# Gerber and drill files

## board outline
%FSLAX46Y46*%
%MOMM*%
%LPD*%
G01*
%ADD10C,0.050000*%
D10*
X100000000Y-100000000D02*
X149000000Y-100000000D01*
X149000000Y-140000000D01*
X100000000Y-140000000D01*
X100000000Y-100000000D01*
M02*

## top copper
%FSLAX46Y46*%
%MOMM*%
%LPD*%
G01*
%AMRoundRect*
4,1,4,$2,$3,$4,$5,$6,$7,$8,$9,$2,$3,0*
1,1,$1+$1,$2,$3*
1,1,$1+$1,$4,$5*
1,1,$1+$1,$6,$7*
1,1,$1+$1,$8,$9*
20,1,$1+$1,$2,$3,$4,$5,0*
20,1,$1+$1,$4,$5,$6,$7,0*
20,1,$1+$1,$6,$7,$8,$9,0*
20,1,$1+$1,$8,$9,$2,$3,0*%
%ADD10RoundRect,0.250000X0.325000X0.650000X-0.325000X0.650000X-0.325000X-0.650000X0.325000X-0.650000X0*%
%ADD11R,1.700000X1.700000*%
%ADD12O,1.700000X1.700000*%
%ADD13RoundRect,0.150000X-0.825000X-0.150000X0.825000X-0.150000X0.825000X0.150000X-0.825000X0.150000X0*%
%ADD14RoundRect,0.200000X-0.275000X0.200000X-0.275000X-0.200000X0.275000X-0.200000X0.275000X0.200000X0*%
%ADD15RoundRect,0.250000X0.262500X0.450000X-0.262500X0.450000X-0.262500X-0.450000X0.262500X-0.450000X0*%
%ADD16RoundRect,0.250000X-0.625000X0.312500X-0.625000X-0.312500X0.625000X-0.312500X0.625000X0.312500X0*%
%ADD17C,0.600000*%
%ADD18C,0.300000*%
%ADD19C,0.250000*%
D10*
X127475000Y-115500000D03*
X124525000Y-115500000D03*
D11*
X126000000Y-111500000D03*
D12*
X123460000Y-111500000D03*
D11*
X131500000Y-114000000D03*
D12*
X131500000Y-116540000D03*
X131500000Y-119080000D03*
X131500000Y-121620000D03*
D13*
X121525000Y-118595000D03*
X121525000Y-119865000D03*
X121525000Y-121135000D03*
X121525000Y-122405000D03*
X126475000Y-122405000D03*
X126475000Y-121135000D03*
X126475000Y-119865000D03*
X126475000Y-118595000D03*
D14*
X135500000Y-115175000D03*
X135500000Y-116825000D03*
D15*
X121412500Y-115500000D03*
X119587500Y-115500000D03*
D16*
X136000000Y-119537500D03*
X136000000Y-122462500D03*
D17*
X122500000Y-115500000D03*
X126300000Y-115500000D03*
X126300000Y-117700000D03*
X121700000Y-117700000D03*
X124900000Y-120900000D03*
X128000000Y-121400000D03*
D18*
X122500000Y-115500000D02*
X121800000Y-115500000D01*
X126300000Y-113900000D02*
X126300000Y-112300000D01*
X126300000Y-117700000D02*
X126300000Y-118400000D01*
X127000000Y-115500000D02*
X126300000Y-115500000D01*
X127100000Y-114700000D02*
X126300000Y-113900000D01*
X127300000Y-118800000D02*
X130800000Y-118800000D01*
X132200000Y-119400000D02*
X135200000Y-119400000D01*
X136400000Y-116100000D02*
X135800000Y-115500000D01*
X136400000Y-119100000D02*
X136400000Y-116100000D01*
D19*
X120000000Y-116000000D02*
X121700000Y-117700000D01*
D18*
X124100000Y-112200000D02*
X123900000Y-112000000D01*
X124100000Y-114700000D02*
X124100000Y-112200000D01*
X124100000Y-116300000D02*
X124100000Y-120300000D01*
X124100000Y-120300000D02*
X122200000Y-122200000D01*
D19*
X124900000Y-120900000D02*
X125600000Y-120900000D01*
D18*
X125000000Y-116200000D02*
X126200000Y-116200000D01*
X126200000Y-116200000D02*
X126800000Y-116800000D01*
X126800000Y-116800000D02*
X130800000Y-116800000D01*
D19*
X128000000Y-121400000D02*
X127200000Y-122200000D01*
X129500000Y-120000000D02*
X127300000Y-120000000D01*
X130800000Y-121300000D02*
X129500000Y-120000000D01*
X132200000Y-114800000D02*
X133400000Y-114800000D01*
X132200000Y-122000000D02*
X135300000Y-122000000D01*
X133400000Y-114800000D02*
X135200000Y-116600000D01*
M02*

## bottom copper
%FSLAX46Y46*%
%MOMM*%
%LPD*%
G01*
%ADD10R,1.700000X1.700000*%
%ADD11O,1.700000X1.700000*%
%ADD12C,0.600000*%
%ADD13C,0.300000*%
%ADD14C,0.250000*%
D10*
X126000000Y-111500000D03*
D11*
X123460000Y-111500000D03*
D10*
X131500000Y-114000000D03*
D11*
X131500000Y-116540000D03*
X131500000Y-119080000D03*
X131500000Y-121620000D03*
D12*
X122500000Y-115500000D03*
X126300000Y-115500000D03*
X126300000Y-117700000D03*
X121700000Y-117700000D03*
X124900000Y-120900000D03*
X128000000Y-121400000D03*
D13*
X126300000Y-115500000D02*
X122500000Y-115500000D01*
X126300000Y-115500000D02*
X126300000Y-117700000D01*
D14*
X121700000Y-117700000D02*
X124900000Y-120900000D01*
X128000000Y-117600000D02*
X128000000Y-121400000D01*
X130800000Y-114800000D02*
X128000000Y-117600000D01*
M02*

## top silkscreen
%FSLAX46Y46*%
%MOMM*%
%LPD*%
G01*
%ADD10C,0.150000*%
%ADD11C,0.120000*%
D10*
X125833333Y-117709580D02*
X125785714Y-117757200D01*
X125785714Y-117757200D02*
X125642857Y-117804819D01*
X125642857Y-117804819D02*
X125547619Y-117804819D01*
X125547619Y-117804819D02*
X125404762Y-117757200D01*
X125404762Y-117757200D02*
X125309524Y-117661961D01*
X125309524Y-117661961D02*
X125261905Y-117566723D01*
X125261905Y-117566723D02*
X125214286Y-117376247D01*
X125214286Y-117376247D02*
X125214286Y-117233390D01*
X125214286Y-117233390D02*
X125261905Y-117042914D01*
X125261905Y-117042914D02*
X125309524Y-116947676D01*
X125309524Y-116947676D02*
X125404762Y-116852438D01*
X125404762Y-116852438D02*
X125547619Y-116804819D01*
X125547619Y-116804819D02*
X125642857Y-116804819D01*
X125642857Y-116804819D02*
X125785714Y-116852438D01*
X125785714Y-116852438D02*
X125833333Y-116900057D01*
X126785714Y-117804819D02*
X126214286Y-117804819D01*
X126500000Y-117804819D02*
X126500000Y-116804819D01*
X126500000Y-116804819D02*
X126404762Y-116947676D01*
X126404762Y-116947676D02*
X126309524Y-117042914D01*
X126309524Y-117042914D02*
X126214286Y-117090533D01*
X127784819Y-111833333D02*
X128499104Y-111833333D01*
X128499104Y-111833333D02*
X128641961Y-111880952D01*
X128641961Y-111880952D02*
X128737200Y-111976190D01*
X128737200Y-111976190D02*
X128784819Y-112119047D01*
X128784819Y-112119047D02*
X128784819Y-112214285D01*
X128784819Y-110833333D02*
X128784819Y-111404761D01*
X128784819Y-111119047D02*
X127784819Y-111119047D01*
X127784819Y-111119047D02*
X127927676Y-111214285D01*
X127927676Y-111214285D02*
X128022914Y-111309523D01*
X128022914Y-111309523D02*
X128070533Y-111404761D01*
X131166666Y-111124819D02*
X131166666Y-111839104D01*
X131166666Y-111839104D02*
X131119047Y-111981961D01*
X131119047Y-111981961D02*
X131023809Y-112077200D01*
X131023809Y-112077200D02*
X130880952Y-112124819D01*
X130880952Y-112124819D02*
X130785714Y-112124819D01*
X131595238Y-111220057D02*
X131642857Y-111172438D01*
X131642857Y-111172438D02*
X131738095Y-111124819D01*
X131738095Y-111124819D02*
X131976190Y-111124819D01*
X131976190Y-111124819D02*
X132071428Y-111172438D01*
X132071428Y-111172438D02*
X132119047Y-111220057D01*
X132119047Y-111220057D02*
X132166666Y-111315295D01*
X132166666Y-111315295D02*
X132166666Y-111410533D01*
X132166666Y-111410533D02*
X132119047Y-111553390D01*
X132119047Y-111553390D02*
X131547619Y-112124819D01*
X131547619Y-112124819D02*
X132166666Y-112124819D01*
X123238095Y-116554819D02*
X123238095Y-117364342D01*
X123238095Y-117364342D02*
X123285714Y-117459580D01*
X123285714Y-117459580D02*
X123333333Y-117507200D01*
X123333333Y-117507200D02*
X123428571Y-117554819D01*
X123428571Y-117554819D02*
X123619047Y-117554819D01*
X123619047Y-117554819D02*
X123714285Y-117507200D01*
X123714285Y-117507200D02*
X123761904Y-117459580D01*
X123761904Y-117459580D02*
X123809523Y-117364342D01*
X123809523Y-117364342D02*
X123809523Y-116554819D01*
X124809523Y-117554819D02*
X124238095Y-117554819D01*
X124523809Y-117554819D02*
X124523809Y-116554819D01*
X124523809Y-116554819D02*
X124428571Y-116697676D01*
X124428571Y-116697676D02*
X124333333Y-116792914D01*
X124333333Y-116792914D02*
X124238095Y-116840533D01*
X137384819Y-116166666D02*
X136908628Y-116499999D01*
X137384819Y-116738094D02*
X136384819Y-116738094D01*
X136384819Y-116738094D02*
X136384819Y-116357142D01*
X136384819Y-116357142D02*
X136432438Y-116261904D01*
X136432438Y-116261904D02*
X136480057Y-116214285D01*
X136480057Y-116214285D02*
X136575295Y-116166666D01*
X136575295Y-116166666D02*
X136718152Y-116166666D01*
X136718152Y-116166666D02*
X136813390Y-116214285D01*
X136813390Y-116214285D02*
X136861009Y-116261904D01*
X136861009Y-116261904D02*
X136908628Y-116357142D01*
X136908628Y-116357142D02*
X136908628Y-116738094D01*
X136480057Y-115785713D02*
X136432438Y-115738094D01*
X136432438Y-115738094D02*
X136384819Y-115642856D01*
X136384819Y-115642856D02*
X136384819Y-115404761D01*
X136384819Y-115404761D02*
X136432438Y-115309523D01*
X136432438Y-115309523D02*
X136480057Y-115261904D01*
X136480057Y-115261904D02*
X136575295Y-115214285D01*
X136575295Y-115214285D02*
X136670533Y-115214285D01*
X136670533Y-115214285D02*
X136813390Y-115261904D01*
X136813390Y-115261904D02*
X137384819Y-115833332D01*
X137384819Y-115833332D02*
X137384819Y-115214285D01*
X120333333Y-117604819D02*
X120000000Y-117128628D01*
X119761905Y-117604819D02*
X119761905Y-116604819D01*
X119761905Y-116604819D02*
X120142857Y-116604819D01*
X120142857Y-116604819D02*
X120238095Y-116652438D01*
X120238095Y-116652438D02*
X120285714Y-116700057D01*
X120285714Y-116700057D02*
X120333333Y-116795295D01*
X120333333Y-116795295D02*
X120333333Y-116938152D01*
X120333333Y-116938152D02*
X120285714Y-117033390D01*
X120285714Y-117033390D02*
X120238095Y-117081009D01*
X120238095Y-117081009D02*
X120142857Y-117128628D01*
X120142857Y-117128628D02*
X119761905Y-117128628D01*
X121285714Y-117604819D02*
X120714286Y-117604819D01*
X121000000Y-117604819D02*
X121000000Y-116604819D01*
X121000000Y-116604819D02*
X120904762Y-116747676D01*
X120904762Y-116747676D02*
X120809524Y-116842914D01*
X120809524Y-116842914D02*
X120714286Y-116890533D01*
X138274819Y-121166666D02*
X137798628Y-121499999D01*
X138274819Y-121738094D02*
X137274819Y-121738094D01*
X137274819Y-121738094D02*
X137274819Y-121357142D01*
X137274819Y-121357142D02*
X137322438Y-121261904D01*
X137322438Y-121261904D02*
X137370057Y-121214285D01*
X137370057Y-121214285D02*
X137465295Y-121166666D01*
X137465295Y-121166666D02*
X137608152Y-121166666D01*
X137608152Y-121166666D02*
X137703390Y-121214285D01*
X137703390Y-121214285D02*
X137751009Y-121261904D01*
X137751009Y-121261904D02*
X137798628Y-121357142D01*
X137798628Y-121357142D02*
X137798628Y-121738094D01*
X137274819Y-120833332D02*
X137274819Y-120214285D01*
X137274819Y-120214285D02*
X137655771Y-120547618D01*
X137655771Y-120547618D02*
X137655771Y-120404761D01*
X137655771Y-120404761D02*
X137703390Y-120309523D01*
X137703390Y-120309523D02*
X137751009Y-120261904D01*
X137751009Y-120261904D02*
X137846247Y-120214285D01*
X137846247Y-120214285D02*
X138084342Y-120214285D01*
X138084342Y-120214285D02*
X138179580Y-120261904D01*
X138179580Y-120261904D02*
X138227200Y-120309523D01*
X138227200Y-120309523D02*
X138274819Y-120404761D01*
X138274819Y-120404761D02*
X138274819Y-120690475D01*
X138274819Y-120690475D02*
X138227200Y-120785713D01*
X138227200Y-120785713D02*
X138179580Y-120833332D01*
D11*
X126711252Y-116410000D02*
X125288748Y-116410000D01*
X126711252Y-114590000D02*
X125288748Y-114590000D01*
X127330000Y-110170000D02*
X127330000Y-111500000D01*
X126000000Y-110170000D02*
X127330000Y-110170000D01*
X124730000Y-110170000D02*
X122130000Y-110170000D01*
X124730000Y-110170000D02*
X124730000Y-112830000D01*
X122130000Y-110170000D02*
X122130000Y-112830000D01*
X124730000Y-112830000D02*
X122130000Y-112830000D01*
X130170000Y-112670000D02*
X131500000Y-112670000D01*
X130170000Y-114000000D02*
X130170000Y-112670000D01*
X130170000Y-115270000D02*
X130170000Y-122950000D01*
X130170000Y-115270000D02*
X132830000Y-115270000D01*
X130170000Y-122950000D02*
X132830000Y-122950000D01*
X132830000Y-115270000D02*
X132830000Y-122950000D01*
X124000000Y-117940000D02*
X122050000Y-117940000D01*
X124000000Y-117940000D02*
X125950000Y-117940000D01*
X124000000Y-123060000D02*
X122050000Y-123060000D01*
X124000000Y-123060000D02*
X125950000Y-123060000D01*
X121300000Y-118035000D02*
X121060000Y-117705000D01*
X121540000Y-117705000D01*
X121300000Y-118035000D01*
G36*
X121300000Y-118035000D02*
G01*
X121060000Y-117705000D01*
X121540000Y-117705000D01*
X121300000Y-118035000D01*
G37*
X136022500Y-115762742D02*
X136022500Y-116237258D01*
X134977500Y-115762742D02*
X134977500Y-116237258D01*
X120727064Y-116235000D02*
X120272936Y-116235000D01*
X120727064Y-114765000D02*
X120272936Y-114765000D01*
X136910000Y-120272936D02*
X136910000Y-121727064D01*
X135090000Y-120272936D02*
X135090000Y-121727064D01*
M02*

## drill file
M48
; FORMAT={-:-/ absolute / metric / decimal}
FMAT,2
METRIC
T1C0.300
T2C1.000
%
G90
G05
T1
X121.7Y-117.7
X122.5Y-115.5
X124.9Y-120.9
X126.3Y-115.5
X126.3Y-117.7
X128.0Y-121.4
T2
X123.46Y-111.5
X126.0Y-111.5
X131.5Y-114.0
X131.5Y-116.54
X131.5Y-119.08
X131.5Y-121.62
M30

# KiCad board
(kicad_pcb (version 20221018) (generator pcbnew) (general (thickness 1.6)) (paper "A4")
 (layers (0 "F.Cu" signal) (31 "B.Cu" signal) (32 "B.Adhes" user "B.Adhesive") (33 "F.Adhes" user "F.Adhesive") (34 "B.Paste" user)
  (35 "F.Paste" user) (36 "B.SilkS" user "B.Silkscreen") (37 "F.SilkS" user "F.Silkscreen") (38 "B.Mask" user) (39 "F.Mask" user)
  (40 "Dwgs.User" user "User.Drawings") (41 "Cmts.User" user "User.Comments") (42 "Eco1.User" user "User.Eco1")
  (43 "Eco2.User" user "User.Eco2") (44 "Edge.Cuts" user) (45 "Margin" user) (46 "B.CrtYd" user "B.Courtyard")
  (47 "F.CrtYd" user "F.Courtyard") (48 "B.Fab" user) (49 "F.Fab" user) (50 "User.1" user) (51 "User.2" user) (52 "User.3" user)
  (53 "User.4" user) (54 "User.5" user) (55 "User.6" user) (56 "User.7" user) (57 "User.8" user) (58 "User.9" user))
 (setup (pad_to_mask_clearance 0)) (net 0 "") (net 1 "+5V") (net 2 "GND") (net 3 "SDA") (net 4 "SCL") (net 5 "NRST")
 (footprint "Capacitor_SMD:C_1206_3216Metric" (layer "F.Cu") (at 126 115.5 180)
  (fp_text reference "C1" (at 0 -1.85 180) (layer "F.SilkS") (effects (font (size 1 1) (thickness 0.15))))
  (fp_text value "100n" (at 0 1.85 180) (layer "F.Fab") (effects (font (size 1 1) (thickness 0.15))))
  (fp_line (start -0.711252 -0.91) (end 0.711252 -0.91) (stroke (width 0.12) (type solid)) (layer "F.SilkS"))
  (fp_line (start -0.711252 0.91) (end 0.711252 0.91) (stroke (width 0.12) (type solid)) (layer "F.SilkS"))
  (pad "1" smd roundrect (at -1.475 0 180) (size 1.15 1.8) (layers "F.Cu" "F.Paste" "F.Mask") (roundrect_rratio 0.217391) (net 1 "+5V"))
  (pad "2" smd roundrect (at 1.475 0 180) (size 1.15 1.8) (layers "F.Cu" "F.Paste" "F.Mask") (roundrect_rratio 0.217391) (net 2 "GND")))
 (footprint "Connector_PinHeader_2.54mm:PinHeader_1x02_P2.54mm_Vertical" (layer "F.Cu") (at 126 111.5 -90)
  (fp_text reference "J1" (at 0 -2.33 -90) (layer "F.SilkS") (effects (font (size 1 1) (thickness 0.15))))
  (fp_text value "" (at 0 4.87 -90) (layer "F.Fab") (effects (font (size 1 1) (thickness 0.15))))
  (fp_line (start -1.33 -1.33) (end 0 -1.33) (stroke (width 0.12) (type solid)) (layer "F.SilkS"))
  (fp_line (start -1.33 0) (end -1.33 -1.33) (stroke (width 0.12) (type solid)) (layer "F.SilkS"))
  (fp_line (start -1.33 1.27) (end -1.33 3.87) (stroke (width 0.12) (type solid)) (layer "F.SilkS"))
  (fp_line (start -1.33 1.27) (end 1.33 1.27) (stroke (width 0.12) (type solid)) (layer "F.SilkS"))
  (fp_line (start -1.33 3.87) (end 1.33 3.87) (stroke (width 0.12) (type solid)) (layer "F.SilkS"))
  (fp_line (start 1.33 1.27) (end 1.33 3.87) (stroke (width 0.12) (type solid)) (layer "F.SilkS"))
  (pad "1" thru_hole rect (at 0 0 270) (size 1.7 1.7) (drill 1) (layers "*.Cu" "*.Mask") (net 1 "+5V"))
  (pad "2" thru_hole oval (at 0 2.54 270) (size 1.7 1.7) (drill 1) (layers "*.Cu" "*.Mask") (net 2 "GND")))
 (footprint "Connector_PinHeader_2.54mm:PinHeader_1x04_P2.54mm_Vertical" (layer "F.Cu") (at 131.5 114)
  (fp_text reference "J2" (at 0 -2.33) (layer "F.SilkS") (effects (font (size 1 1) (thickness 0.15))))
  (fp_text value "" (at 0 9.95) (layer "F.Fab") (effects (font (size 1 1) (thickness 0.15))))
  (fp_line (start -1.33 -1.33) (end 0 -1.33) (stroke (width 0.12) (type solid)) (layer "F.SilkS"))
  (fp_line (start -1.33 0) (end -1.33 -1.33) (stroke (width 0.12) (type solid)) (layer "F.SilkS"))
  (fp_line (start -1.33 1.27) (end -1.33 8.95) (stroke (width 0.12) (type solid)) (layer "F.SilkS"))
  (fp_line (start -1.33 1.27) (end 1.33 1.27) (stroke (width 0.12) (type solid)) (layer "F.SilkS"))
  (fp_line (start -1.33 8.95) (end 1.33 8.95) (stroke (width 0.12) (type solid)) (layer "F.SilkS"))
  (fp_line (start 1.33 1.27) (end 1.33 8.95) (stroke (width 0.12) (type solid)) (layer "F.SilkS"))
  (pad "1" thru_hole rect (at 0 0) (size 1.7 1.7) (drill 1) (layers "*.Cu" "*.Mask") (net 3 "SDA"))
  (pad "2" thru_hole oval (at 0 2.54) (size 1.7 1.7) (drill 1) (layers "*.Cu" "*.Mask") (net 2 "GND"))
  (pad "3" thru_hole oval (at 0 5.08) (size 1.7 1.7) (drill 1) (layers "*.Cu" "*.Mask") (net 1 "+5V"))
  (pad "4" thru_hole oval (at 0 7.62) (size 1.7 1.7) (drill 1) (layers "*.Cu" "*.Mask") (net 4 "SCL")))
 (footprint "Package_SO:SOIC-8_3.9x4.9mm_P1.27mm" (layer "F.Cu") (at 124 120.5)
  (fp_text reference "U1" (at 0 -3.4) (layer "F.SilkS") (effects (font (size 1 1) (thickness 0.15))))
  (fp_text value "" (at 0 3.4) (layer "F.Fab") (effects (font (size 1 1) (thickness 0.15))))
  (fp_line (start 0 -2.56) (end -1.95 -2.56) (stroke (width 0.12) (type solid)) (layer "F.SilkS"))
  (fp_line (start 0 -2.56) (end 1.95 -2.56) (stroke (width 0.12) (type solid)) (layer "F.SilkS"))
  (fp_line (start 0 2.56) (end -1.95 2.56) (stroke (width 0.12) (type solid)) (layer "F.SilkS"))
  (fp_line (start 0 2.56) (end 1.95 2.56) (stroke (width 0.12) (type solid)) (layer "F.SilkS"))
  (fp_poly
   (pts (xy -2.7 -2.465) (xy -2.94 -2.795) (xy -2.46 -2.795) (xy -2.7 -2.465)) (stroke (width 0.12) (type solid)) (fill solid)
   (layer "F.SilkS"))
  (pad "1" smd roundrect (at -2.475 -1.905) (size 1.95 0.6) (layers "F.Cu" "F.Paste" "F.Mask") (roundrect_rratio 0.25))
  (pad "2" smd roundrect (at -2.475 -0.635) (size 1.95 0.6) (layers "F.Cu" "F.Paste" "F.Mask") (roundrect_rratio 0.25))
  (pad "3" smd roundrect (at -2.475 0.635) (size 1.95 0.6) (layers "F.Cu" "F.Paste" "F.Mask") (roundrect_rratio 0.25))
  (pad "4" smd roundrect (at -2.475 1.905) (size 1.95 0.6) (layers "F.Cu" "F.Paste" "F.Mask") (roundrect_rratio 0.25) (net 2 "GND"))
  (pad "5" smd roundrect (at 2.475 1.905) (size 1.95 0.6) (layers "F.Cu" "F.Paste" "F.Mask") (roundrect_rratio 0.25) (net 3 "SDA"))
  (pad "6" smd roundrect (at 2.475 0.635) (size 1.95 0.6) (layers "F.Cu" "F.Paste" "F.Mask") (roundrect_rratio 0.25) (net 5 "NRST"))
  (pad "7" smd roundrect (at 2.475 -0.635) (size 1.95 0.6) (layers "F.Cu" "F.Paste" "F.Mask") (roundrect_rratio 0.25) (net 4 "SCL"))
  (pad "8" smd roundrect (at 2.475 -1.905) (size 1.95 0.6) (layers "F.Cu" "F.Paste" "F.Mask") (roundrect_rratio 0.25) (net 1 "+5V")))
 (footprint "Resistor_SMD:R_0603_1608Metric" (layer "F.Cu") (at 135.5 116 -90)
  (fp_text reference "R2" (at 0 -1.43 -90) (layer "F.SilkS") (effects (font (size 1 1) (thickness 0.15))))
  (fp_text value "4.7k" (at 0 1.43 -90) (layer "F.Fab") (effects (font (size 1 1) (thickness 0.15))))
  (fp_line (start -0.237258 -0.5225) (end 0.237258 -0.5225) (stroke (width 0.12) (type solid)) (layer "F.SilkS"))
  (fp_line (start -0.237258 0.5225) (end 0.237258 0.5225) (stroke (width 0.12) (type solid)) (layer "F.SilkS"))
  (pad "1" smd roundrect (at -0.825 0 270) (size 0.8 0.95) (layers "F.Cu" "F.Paste" "F.Mask") (roundrect_rratio 0.25) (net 1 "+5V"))
  (pad "2" smd roundrect (at 0.825 0 270) (size 0.8 0.95) (layers "F.Cu" "F.Paste" "F.Mask") (roundrect_rratio 0.25) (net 3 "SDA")))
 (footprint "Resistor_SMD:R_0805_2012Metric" (layer "F.Cu") (at 120.5 115.5 180)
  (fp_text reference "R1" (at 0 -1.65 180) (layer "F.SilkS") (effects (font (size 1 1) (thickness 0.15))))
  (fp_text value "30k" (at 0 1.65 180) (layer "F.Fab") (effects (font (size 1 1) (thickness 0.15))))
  (fp_line (start -0.227064 -0.735) (end 0.227064 -0.735) (stroke (width 0.12) (type solid)) (layer "F.SilkS"))
  (fp_line (start -0.227064 0.735) (end 0.227064 0.735) (stroke (width 0.12) (type solid)) (layer "F.SilkS"))
  (pad "1" smd roundrect (at -0.9125 0 180) (size 1.025 1.4) (layers "F.Cu" "F.Paste" "F.Mask") (roundrect_rratio 0.243902) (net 1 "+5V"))
  (pad "2" smd roundrect (at 0.9125 0 180) (size 1.025 1.4) (layers "F.Cu" "F.Paste" "F.Mask") (roundrect_rratio 0.243902) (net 5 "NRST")))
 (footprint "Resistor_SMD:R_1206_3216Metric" (layer "F.Cu") (at 136 121 -90)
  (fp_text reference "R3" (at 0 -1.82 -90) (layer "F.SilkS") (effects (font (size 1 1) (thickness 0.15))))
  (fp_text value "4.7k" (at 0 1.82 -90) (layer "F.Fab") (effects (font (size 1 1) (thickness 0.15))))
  (fp_line (start -0.727064 -0.91) (end 0.727064 -0.91) (stroke (width 0.12) (type solid)) (layer "F.SilkS"))
  (fp_line (start -0.727064 0.91) (end 0.727064 0.91) (stroke (width 0.12) (type solid)) (layer "F.SilkS"))
  (pad "1" smd roundrect (at -1.4625 0 270) (size 1.125 1.75) (layers "F.Cu" "F.Paste" "F.Mask") (roundrect_rratio 0.222222) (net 1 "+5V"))
  (pad "2" smd roundrect (at 1.4625 0 270) (size 1.125 1.75) (layers "F.Cu" "F.Paste" "F.Mask") (roundrect_rratio 0.222222) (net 4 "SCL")))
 (gr_rect (start 100 100) (end 149 140) (stroke (width 0.05) (type default)) (fill none) (layer "Edge.Cuts"))
 (segment (start 122.5 115.5) (end 121.8 115.5) (width 0.3) (layer "F.Cu") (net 1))
 (segment (start 126.3 113.9) (end 126.3 112.3) (width 0.3) (layer "F.Cu") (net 1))
 (segment (start 126.3 117.7) (end 126.3 118.4) (width 0.3) (layer "F.Cu") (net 1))
 (segment (start 127 115.5) (end 126.3 115.5) (width 0.3) (layer "F.Cu") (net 1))
 (segment (start 127.1 114.7) (end 126.3 113.9) (width 0.3) (layer "F.Cu") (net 1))
 (segment (start 127.3 118.8) (end 130.8 118.8) (width 0.3) (layer "F.Cu") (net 1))
 (segment (start 132.2 119.4) (end 135.2 119.4) (width 0.3) (layer "F.Cu") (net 1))
 (segment (start 136.4 116.1) (end 135.8 115.5) (width 0.3) (layer "F.Cu") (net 1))
 (segment (start 136.4 119.1) (end 136.4 116.1) (width 0.3) (layer "F.Cu") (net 1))
 (via (at 122.5 115.5) (size 0.6) (drill 0.3) (layers "F.Cu" "B.Cu") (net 1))
 (via (at 126.3 115.5) (size 0.6) (drill 0.3) (layers "F.Cu" "B.Cu") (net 1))
 (via (at 126.3 117.7) (size 0.6) (drill 0.3) (layers "F.Cu" "B.Cu") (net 1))
 (segment (start 120 116) (end 121.7 117.7) (width 0.25) (layer "F.Cu") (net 5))
 (segment (start 124.1 112.2) (end 123.9 112) (width 0.3) (layer "F.Cu") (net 2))
 (segment (start 124.1 114.7) (end 124.1 112.2) (width 0.3) (layer "F.Cu") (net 2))
 (segment (start 124.1 116.3) (end 124.1 120.3) (width 0.3) (layer "F.Cu") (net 2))
 (segment (start 124.1 120.3) (end 122.2 122.2) (width 0.3) (layer "F.Cu") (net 2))
 (segment (start 124.9 120.9) (end 125.6 120.9) (width 0.25) (layer "F.Cu") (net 5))
 (segment (start 125 116.2) (end 126.2 116.2) (width 0.3) (layer "F.Cu") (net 2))
 (segment (start 126.2 116.2) (end 126.8 116.8) (width 0.3) (layer "F.Cu") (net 2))
 (segment (start 126.3 115.5) (end 122.5 115.5) (width 0.3) (layer "B.Cu") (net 1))
 (segment (start 126.3 115.5) (end 126.3 117.7) (width 0.3) (layer "B.Cu") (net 1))
 (segment (start 126.8 116.8) (end 130.8 116.8) (width 0.3) (layer "F.Cu") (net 2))
 (via (at 121.7 117.7) (size 0.6) (drill 0.3) (layers "F.Cu" "B.Cu") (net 5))
 (via (at 124.9 120.9) (size 0.6) (drill 0.3) (layers "F.Cu" "B.Cu") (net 5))
 (segment (start 121.7 117.7) (end 124.9 120.9) (width 0.25) (layer "B.Cu") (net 5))
 (segment (start 128 121.4) (end 127.2 122.2) (width 0.25) (layer "F.Cu") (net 3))
 (segment (start 129.5 120) (end 127.3 120) (width 0.25) (layer "F.Cu") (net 4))
 (segment (start 130.8 121.3) (end 129.5 120) (width 0.25) (layer "F.Cu") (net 4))
 (segment (start 132.2 114.8) (end 133.4 114.8) (width 0.25) (layer "F.Cu") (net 3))
 (segment (start 132.2 122) (end 135.3 122) (width 0.25) (layer "F.Cu") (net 4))
 (segment (start 133.4 114.8) (end 135.2 116.6) (width 0.25) (layer "F.Cu") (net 3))
 (via (at 128 121.4) (size 0.6) (drill 0.3) (layers "F.Cu" "B.Cu") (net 3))
 (segment (start 128 117.6) (end 128 121.4) (width 0.25) (layer "B.Cu") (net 3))
 (segment (start 130.8 114.8) (end 128 117.6) (width 0.25) (layer "B.Cu") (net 3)))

